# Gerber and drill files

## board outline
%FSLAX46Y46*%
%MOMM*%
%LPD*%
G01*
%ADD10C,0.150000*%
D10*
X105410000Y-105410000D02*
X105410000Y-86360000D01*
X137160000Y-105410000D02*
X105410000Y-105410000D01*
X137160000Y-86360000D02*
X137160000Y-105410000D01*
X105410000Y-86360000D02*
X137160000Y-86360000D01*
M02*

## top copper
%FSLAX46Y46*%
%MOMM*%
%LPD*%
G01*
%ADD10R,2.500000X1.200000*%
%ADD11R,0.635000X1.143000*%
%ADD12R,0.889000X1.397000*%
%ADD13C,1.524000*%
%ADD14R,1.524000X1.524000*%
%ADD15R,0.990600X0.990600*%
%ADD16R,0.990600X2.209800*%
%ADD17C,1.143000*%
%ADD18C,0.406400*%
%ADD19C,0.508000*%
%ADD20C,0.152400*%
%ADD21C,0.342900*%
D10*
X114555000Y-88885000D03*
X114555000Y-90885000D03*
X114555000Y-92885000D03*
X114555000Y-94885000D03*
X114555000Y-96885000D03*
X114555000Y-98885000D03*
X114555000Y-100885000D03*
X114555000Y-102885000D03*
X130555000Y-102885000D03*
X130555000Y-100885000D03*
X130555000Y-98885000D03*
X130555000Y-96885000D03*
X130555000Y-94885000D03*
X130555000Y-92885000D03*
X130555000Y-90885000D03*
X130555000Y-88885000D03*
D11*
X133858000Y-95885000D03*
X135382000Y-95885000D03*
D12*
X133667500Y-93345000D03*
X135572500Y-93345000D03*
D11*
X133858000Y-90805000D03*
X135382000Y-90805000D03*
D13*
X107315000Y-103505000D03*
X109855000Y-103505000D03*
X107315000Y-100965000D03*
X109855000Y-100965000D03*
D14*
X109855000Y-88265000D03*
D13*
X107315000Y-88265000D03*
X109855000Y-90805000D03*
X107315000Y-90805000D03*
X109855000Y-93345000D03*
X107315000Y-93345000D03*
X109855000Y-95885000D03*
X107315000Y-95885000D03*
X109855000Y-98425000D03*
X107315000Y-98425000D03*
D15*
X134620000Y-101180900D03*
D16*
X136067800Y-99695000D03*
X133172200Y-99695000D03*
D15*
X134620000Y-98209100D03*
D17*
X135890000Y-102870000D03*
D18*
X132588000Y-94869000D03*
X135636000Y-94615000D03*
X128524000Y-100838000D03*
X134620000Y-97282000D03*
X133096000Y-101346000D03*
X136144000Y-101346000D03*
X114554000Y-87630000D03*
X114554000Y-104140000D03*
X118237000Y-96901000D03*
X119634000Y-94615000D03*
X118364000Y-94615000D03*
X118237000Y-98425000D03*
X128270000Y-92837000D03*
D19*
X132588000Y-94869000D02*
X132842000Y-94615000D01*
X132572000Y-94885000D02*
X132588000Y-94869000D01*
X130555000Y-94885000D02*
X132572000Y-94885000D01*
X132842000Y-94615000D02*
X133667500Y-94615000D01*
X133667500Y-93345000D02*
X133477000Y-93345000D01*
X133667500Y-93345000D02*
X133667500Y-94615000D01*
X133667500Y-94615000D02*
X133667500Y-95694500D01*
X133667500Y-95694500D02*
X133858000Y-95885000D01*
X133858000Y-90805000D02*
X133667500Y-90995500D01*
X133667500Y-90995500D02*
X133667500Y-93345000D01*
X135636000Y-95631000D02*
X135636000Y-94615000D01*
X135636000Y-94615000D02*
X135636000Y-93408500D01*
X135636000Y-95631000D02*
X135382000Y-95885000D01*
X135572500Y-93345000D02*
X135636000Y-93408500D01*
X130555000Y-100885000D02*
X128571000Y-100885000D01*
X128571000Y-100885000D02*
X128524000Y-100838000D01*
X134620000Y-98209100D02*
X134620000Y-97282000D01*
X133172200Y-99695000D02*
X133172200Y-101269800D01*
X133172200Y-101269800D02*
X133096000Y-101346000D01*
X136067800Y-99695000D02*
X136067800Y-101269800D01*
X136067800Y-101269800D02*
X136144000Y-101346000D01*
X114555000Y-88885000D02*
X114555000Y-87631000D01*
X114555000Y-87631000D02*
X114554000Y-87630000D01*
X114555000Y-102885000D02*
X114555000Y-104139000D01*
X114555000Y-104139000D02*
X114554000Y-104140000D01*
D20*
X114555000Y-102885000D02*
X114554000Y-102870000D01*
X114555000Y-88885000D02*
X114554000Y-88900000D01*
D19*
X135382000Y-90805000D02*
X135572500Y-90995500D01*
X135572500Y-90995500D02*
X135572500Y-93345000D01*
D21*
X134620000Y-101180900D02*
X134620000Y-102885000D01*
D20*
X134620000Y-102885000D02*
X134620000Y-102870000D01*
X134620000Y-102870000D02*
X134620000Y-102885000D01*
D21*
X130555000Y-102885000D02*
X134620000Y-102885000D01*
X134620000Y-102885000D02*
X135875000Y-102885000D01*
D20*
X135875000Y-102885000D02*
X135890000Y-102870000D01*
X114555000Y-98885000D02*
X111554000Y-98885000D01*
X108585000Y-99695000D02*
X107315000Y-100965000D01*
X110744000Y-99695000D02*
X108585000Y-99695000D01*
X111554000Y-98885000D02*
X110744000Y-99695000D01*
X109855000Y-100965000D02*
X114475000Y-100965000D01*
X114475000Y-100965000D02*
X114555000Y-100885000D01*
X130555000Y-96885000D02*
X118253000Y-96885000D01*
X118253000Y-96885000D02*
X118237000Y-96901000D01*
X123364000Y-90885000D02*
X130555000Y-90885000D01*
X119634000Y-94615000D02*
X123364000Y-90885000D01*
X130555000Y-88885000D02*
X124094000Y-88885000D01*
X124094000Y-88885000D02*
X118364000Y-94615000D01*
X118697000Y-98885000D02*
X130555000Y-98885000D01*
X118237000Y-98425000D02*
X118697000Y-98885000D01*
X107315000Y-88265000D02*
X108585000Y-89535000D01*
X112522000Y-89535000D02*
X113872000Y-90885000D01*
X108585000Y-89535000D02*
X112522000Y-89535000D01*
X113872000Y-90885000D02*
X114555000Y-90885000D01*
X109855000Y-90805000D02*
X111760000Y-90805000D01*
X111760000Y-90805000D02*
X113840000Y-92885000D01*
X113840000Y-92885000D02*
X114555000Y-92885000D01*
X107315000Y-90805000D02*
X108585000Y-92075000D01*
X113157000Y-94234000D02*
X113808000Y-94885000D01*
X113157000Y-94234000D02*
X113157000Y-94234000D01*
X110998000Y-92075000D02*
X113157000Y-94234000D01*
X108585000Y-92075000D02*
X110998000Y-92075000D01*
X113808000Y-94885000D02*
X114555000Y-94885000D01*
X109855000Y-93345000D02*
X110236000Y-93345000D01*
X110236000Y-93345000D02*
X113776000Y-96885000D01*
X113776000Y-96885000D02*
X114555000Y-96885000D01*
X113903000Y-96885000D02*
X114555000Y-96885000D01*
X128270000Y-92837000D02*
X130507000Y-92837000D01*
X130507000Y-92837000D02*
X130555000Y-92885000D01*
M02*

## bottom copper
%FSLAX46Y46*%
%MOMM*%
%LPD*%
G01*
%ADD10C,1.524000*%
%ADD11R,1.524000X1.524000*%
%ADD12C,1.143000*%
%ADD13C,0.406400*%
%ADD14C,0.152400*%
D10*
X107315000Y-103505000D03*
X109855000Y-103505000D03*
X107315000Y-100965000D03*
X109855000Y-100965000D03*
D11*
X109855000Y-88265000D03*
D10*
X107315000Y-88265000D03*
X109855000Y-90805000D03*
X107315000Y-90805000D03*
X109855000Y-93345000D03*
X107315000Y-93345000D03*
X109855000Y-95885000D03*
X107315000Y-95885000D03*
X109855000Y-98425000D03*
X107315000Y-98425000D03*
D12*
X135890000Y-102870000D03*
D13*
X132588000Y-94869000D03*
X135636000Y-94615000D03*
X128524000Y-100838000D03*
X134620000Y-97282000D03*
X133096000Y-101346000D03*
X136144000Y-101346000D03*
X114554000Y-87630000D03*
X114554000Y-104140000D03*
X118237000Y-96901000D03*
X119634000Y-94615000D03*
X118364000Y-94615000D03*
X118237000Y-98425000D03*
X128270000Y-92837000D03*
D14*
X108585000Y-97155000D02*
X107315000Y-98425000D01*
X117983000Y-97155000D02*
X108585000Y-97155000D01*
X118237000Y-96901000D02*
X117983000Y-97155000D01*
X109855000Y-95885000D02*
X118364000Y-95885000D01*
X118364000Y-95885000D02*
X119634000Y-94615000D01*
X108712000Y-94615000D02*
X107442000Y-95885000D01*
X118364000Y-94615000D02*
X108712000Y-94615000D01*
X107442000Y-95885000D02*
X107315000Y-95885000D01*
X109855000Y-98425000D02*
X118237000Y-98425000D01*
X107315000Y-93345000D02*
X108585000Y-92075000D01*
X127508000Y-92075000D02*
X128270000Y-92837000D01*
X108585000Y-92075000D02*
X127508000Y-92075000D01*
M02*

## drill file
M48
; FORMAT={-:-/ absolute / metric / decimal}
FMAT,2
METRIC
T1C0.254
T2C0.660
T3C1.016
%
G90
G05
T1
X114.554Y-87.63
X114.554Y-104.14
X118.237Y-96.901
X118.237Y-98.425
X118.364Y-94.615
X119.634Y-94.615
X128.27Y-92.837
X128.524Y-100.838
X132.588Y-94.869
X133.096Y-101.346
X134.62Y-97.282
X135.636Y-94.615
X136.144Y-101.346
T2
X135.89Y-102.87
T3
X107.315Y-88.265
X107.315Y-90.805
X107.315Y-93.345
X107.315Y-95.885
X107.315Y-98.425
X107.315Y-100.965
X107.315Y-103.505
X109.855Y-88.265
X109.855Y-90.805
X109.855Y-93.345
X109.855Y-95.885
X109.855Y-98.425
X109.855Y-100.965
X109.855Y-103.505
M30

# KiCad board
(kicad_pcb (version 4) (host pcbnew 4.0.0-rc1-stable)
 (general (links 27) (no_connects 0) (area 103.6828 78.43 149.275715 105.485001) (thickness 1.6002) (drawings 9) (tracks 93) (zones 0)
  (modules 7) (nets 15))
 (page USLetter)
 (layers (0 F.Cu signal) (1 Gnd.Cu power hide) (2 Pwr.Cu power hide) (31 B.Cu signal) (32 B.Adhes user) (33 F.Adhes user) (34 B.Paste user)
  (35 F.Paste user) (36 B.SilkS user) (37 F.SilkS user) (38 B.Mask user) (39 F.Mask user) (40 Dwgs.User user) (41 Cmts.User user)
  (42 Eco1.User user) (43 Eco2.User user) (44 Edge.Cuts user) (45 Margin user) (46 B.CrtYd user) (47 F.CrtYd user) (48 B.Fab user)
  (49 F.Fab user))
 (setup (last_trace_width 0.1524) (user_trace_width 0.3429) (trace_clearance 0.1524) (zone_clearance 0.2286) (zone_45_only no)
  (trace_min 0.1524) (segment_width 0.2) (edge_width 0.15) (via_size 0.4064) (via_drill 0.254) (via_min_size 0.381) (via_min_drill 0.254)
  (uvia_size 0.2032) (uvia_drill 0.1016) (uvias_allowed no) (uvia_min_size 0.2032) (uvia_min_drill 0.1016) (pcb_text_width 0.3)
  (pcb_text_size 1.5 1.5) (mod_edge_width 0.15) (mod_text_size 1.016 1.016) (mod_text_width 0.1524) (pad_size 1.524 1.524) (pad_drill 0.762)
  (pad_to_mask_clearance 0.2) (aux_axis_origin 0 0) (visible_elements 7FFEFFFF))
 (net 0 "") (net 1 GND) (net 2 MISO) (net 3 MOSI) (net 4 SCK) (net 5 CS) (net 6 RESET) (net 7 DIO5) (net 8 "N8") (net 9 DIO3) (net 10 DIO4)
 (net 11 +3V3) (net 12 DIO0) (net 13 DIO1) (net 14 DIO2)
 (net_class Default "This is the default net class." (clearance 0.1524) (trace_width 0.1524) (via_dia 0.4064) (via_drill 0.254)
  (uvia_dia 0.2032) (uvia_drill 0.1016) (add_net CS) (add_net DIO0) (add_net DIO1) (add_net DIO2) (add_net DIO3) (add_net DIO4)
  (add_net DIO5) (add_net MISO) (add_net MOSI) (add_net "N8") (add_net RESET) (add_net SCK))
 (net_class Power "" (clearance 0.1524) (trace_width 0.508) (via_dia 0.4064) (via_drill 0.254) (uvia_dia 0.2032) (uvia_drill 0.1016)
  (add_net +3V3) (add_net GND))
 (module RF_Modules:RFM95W (layer F.Cu) (at 122.555 95.885)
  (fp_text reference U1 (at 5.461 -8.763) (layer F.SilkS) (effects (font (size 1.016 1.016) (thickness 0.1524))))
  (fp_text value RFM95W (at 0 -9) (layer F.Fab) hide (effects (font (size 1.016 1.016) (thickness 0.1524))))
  (pad 1 smd rect (at -8 -7) (size 2.5 1.2) (layers F.Cu F.Paste F.Mask) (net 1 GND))
  (pad 2 smd rect (at -8 -5) (size 2.5 1.2) (layers F.Cu F.Paste F.Mask) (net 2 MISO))
  (pad 3 smd rect (at -8 -3) (size 2.5 1.2) (layers F.Cu F.Paste F.Mask) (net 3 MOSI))
  (pad 4 smd rect (at -8 -1) (size 2.5 1.2) (layers F.Cu F.Paste F.Mask) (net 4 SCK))
  (pad 5 smd rect (at -8 1) (size 2.5 1.2) (layers F.Cu F.Paste F.Mask) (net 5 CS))
  (pad 6 smd rect (at -8 3) (size 2.5 1.2) (layers F.Cu F.Paste F.Mask) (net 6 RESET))
  (pad 7 smd rect (at -8 5) (size 2.5 1.2) (layers F.Cu F.Paste F.Mask) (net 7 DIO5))
  (pad 8 smd rect (at -8 7) (size 2.5 1.2) (layers F.Cu F.Paste F.Mask) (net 1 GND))
  (pad 9 smd rect (at 8 7) (size 2.5 1.2) (layers F.Cu F.Paste F.Mask) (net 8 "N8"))
  (pad 10 smd rect (at 8 5) (size 2.5 1.2) (layers F.Cu F.Paste F.Mask) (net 1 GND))
  (pad 11 smd rect (at 8 3) (size 2.5 1.2) (layers F.Cu F.Paste F.Mask) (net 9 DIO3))
  (pad 12 smd rect (at 8 1) (size 2.5 1.2) (layers F.Cu F.Paste F.Mask) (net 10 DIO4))
  (pad 13 smd rect (at 8 -1) (size 2.5 1.2) (layers F.Cu F.Paste F.Mask) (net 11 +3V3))
  (pad 14 smd rect (at 8 -3) (size 2.5 1.2) (layers F.Cu F.Paste F.Mask) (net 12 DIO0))
  (pad 15 smd rect (at 8 -5) (size 2.5 1.2) (layers F.Cu F.Paste F.Mask) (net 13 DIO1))
  (pad 16 smd rect (at 8 -7) (size 2.5 1.2) (layers F.Cu F.Paste F.Mask) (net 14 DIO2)))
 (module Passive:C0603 (layer F.Cu) (at 134.62 95.885)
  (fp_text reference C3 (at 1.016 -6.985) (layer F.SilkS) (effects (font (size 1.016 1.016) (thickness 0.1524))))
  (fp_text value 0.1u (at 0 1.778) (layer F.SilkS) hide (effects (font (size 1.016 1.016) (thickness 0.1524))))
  (pad 1 smd rect (at -0.762 0) (size 0.635 1.143) (layers F.Cu F.Paste F.Mask) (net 11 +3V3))
  (pad 2 smd rect (at 0.762 0) (size 0.635 1.143) (layers F.Cu F.Paste F.Mask) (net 1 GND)))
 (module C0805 (layer F.Cu) (at 134.62 93.345)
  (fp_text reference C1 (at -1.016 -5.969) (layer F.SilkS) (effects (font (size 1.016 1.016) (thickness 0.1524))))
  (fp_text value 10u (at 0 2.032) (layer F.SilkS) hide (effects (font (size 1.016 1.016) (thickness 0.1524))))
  (pad 1 smd rect (at -0.9525 0) (size 0.889 1.397) (layers F.Cu F.Paste F.Mask) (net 11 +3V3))
  (pad 2 smd rect (at 0.9525 0) (size 0.889 1.397) (layers F.Cu F.Paste F.Mask) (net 1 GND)))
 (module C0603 (layer F.Cu) (at 134.62 90.805)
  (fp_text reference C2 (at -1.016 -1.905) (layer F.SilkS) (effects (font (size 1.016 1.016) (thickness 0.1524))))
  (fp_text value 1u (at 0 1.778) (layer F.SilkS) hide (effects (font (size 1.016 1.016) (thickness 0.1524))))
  (pad 1 smd rect (at -0.762 0) (size 0.635 1.143) (layers F.Cu F.Paste F.Mask) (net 11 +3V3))
  (pad 2 smd rect (at 0.762 0) (size 0.635 1.143) (layers F.Cu F.Paste F.Mask) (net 1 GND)))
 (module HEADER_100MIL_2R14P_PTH (layer B.Cu) (at 108.585 95.885 270)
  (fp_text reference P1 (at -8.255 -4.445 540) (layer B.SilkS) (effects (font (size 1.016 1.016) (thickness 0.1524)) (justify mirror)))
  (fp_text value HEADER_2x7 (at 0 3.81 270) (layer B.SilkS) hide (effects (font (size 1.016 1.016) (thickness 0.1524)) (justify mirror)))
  (pad 14 thru_hole circle (at 7.62 1.27 270) (size 1.524 1.524) (drill 1.016) (layers *.Cu *.Mask B.SilkS) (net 1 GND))
  (pad 13 thru_hole circle (at 7.62 -1.27 270) (size 1.524 1.524) (drill 1.016) (layers *.Cu *.Mask B.SilkS) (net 11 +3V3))
  (pad 12 thru_hole circle (at 5.08 1.27 270) (size 1.524 1.524) (drill 1.016) (layers *.Cu *.Mask B.SilkS) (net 6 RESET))
  (pad 11 thru_hole circle (at 5.08 -1.27 270) (size 1.524 1.524) (drill 1.016) (layers *.Cu *.Mask B.SilkS) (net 7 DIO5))
  (pad 1 thru_hole rect (at -7.62 -1.27 270) (size 1.524 1.524) (drill 1.016) (layers *.Cu *.Mask B.SilkS) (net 1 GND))
  (pad 2 thru_hole circle (at -7.62 1.27 270) (size 1.524 1.524) (drill 1.016) (layers *.Cu *.Mask B.SilkS) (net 2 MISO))
  (pad 3 thru_hole circle (at -5.08 -1.27 270) (size 1.524 1.524) (drill 1.016) (layers *.Cu *.Mask B.SilkS) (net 3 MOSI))
  (pad 4 thru_hole circle (at -5.08 1.27 270) (size 1.524 1.524) (drill 1.016) (layers *.Cu *.Mask B.SilkS) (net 4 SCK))
  (pad 5 thru_hole circle (at -2.54 -1.27 270) (size 1.524 1.524) (drill 1.016) (layers *.Cu *.Mask B.SilkS) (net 5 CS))
  (pad 6 thru_hole circle (at -2.54 1.27 270) (size 1.524 1.524) (drill 1.016) (layers *.Cu *.Mask B.SilkS) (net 12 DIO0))
  (pad 7 thru_hole circle (at 0 -1.27 270) (size 1.524 1.524) (drill 1.016) (layers *.Cu *.Mask B.SilkS) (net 13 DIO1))
  (pad 8 thru_hole circle (at 0 1.27 270) (size 1.524 1.524) (drill 1.016) (layers *.Cu *.Mask B.SilkS) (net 14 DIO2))
  (pad 9 thru_hole circle (at 2.54 -1.27 270) (size 1.524 1.524) (drill 1.016) (layers *.Cu *.Mask B.SilkS) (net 9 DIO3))
  (pad 10 thru_hole circle (at 2.54 1.27 270) (size 1.524 1.524) (drill 1.016) (layers *.Cu *.Mask B.SilkS) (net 10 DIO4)))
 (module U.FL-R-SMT (layer F.Cu) (at 134.62 99.695)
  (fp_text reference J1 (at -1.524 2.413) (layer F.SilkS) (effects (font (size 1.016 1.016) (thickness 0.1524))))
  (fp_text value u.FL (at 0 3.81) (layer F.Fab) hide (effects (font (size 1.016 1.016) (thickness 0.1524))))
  (pad 1 smd rect (at 0 1.4859) (size 0.9906 0.9906) (layers F.Cu F.Paste F.Mask) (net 8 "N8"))
  (pad 4 smd rect (at 1.4478 0) (size 0.9906 2.2098) (layers F.Cu F.Paste F.Mask) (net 1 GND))
  (pad 2 smd rect (at -1.4478 0) (size 0.9906 2.2098) (layers F.Cu F.Paste F.Mask) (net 1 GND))
  (pad 3 smd rect (at 0 -1.4859) (size 0.9906 0.9906) (layers F.Cu F.Paste F.Mask) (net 1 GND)))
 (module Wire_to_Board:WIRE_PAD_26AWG (layer F.Cu) (at 135.89 102.87)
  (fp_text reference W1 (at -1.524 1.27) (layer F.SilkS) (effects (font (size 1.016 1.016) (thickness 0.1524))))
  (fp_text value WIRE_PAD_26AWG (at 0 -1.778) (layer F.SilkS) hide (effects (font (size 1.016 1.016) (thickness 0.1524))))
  (pad 1 thru_hole circle (at 0 0) (size 1.143 1.143) (drill 0.6604) (layers *.Cu *.Mask F.SilkS) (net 8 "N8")))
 (gr_line (start 105.41 105.41) (end 105.41 86.36) (angle 90) (layer Edge.Cuts) (width 0.15))
 (gr_line (start 137.16 105.41) (end 105.41 105.41) (angle 90) (layer Edge.Cuts) (width 0.15))
 (gr_line (start 137.16 86.36) (end 137.16 105.41) (angle 90) (layer Edge.Cuts) (width 0.15))
 (gr_line (start 105.41 86.36) (end 137.16 86.36) (angle 90) (layer Edge.Cuts) (width 0.15))
 (segment (start 132.588 94.869) (end 132.842 94.615) (width 0.508) (layer F.Cu) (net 11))
 (segment (start 132.572 94.885) (end 132.588 94.869) (width 0.508) (layer F.Cu) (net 11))
 (via (at 132.588 94.869) (size 0.4064) (drill 0.254) (layers F.Cu B.Cu) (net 11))
 (segment (start 130.555 94.885) (end 132.572 94.885) (width 0.508) (layer F.Cu) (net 11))
 (segment (start 132.842 94.615) (end 133.6675 94.615) (width 0.508) (layer F.Cu) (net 11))
 (segment (start 133.6675 93.345) (end 133.477 93.345) (width 0.508) (layer F.Cu) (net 11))
 (segment (start 133.6675 93.345) (end 133.6675 94.615) (width 0.508) (layer F.Cu) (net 11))
 (segment (start 133.6675 94.615) (end 133.6675 95.6945) (width 0.508) (layer F.Cu) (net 11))
 (segment (start 133.6675 95.6945) (end 133.858 95.885) (width 0.508) (layer F.Cu) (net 11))
 (segment (start 133.858 90.805) (end 133.6675 90.9955) (width 0.508) (layer F.Cu) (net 11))
 (segment (start 133.6675 90.9955) (end 133.6675 93.345) (width 0.508) (layer F.Cu) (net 11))
 (segment (start 135.636 95.631) (end 135.636 94.615) (width 0.508) (layer F.Cu) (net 1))
 (via (at 135.636 94.615) (size 0.4064) (drill 0.254) (layers F.Cu B.Cu) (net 1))
 (segment (start 135.636 94.615) (end 135.636 93.4085) (width 0.508) (layer F.Cu) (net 1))
 (segment (start 135.636 95.631) (end 135.382 95.885) (width 0.508) (layer F.Cu) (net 1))
 (segment (start 135.5725 93.345) (end 135.636 93.4085) (width 0.508) (layer F.Cu) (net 1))
 (segment (start 130.555 100.885) (end 128.571 100.885) (width 0.508) (layer F.Cu) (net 1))
 (via (at 128.524 100.838) (size 0.4064) (drill 0.254) (layers F.Cu B.Cu) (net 1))
 (segment (start 128.571 100.885) (end 128.524 100.838) (width 0.508) (layer F.Cu) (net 1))
 (segment (start 134.62 98.2091) (end 134.62 97.282) (width 0.508) (layer F.Cu) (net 1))
 (via (at 134.62 97.282) (size 0.4064) (drill 0.254) (layers F.Cu B.Cu) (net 1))
 (segment (start 133.1722 99.695) (end 133.1722 101.2698) (width 0.508) (layer F.Cu) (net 1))
 (via (at 133.096 101.346) (size 0.4064) (drill 0.254) (layers F.Cu B.Cu) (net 1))
 (segment (start 133.1722 101.2698) (end 133.096 101.346) (width 0.508) (layer F.Cu) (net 1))
 (segment (start 136.0678 99.695) (end 136.0678 101.2698) (width 0.508) (layer F.Cu) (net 1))
 (via (at 136.144 101.346) (size 0.4064) (drill 0.254) (layers F.Cu B.Cu) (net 1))
 (segment (start 136.0678 101.2698) (end 136.144 101.346) (width 0.508) (layer F.Cu) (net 1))
 (segment (start 114.555 88.885) (end 114.555 87.631) (width 0.508) (layer F.Cu) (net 1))
 (via (at 114.554 87.63) (size 0.4064) (drill 0.254) (layers F.Cu B.Cu) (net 1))
 (segment (start 114.555 87.631) (end 114.554 87.63) (width 0.508) (layer F.Cu) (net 1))
 (segment (start 114.555 102.885) (end 114.555 104.139) (width 0.508) (layer F.Cu) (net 1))
 (via (at 114.554 104.14) (size 0.4064) (drill 0.254) (layers F.Cu B.Cu) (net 1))
 (segment (start 114.555 104.139) (end 114.554 104.14) (width 0.508) (layer F.Cu) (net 1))
 (segment (start 114.555 102.885) (end 114.554 102.87) (width 0.1524) (layer F.Cu) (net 1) (status 80000))
 (segment (start 114.555 88.885) (end 114.554 88.9) (width 0.1524) (layer F.Cu) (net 1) (status 80000))
 (segment (start 135.382 90.805) (end 135.5725 90.9955) (width 0.508) (layer F.Cu) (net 1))
 (segment (start 135.5725 90.9955) (end 135.5725 93.345) (width 0.508) (layer F.Cu) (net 1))
 (segment (start 134.62 101.1809) (end 134.62 102.885) (width 0.3429) (layer F.Cu) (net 8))
 (segment (start 134.62 102.885) (end 134.62 102.87) (width 0.1524) (layer F.Cu) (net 8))
 (segment (start 134.62 102.87) (end 134.62 102.885) (width 0.1524) (layer F.Cu) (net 8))
 (segment (start 130.555 102.885) (end 134.62 102.885) (width 0.3429) (layer F.Cu) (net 8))
 (segment (start 134.62 102.885) (end 135.875 102.885) (width 0.3429) (layer F.Cu) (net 8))
 (segment (start 135.875 102.885) (end 135.89 102.87) (width 0.1524) (layer F.Cu) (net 8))
 (segment (start 114.555 98.885) (end 111.554 98.885) (width 0.1524) (layer F.Cu) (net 6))
 (segment (start 108.585 99.695) (end 107.315 100.965) (width 0.1524) (layer F.Cu) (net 6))
 (segment (start 110.744 99.695) (end 108.585 99.695) (width 0.1524) (layer F.Cu) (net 6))
 (segment (start 111.554 98.885) (end 110.744 99.695) (width 0.1524) (layer F.Cu) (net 6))
 (segment (start 109.855 100.965) (end 114.475 100.965) (width 0.1524) (layer F.Cu) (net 7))
 (segment (start 114.475 100.965) (end 114.555 100.885) (width 0.1524) (layer F.Cu) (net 7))
 (segment (start 130.555 96.885) (end 118.253 96.885) (width 0.1524) (layer F.Cu) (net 10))
 (segment (start 108.585 97.155) (end 107.315 98.425) (width 0.1524) (layer B.Cu) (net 10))
 (segment (start 117.983 97.155) (end 108.585 97.155) (width 0.1524) (layer B.Cu) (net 10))
 (segment (start 118.237 96.901) (end 117.983 97.155) (width 0.1524) (layer B.Cu) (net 10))
 (via (at 118.237 96.901) (size 0.4064) (drill 0.254) (layers F.Cu B.Cu) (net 10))
 (segment (start 118.253 96.885) (end 118.237 96.901) (width 0.1524) (layer F.Cu) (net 10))
 (segment (start 109.855 95.885) (end 118.364 95.885) (width 0.1524) (layer B.Cu) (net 13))
 (segment (start 123.364 90.885) (end 130.555 90.885) (width 0.1524) (layer F.Cu) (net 13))
 (segment (start 119.634 94.615) (end 123.364 90.885) (width 0.1524) (layer F.Cu) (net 13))
 (via (at 119.634 94.615) (size 0.4064) (drill 0.254) (layers F.Cu B.Cu) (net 13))
 (segment (start 118.364 95.885) (end 119.634 94.615) (width 0.1524) (layer B.Cu) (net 13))
 (segment (start 130.555 88.885) (end 124.094 88.885) (width 0.1524) (layer F.Cu) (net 14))
 (segment (start 108.712 94.615) (end 107.442 95.885) (width 0.1524) (layer B.Cu) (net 14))
 (segment (start 118.364 94.615) (end 108.712 94.615) (width 0.1524) (layer B.Cu) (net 14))
 (via (at 118.364 94.615) (size 0.4064) (drill 0.254) (layers F.Cu B.Cu) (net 14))
 (segment (start 124.094 88.885) (end 118.364 94.615) (width 0.1524) (layer F.Cu) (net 14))
 (segment (start 107.442 95.885) (end 107.315 95.885) (width 0.1524) (layer B.Cu) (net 14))
 (segment (start 109.855 98.425) (end 118.237 98.425) (width 0.1524) (layer B.Cu) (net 9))
 (segment (start 118.697 98.885) (end 130.555 98.885) (width 0.1524) (layer F.Cu) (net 9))
 (segment (start 118.237 98.425) (end 118.697 98.885) (width 0.1524) (layer F.Cu) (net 9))
 (via (at 118.237 98.425) (size 0.4064) (drill 0.254) (layers F.Cu B.Cu) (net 9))
 (segment (start 107.315 88.265) (end 108.585 89.535) (width 0.1524) (layer F.Cu) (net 2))
 (segment (start 112.522 89.535) (end 113.872 90.885) (width 0.1524) (layer F.Cu) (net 2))
 (segment (start 108.585 89.535) (end 112.522 89.535) (width 0.1524) (layer F.Cu) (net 2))
 (segment (start 113.872 90.885) (end 114.555 90.885) (width 0.1524) (layer F.Cu) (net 2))
 (segment (start 109.855 90.805) (end 111.76 90.805) (width 0.1524) (layer F.Cu) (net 3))
 (segment (start 111.76 90.805) (end 113.84 92.885) (width 0.1524) (layer F.Cu) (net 3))
 (segment (start 113.84 92.885) (end 114.555 92.885) (width 0.1524) (layer F.Cu) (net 3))
 (segment (start 107.315 90.805) (end 108.585 92.075) (width 0.1524) (layer F.Cu) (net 4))
 (segment (start 113.157 94.234) (end 113.808 94.885) (width 0.1524) (layer F.Cu) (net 4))
 (segment (start 113.157 94.234) (end 113.157 94.234) (width 0.1524) (layer F.Cu) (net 4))
 (segment (start 110.998 92.075) (end 113.157 94.234) (width 0.1524) (layer F.Cu) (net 4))
 (segment (start 108.585 92.075) (end 110.998 92.075) (width 0.1524) (layer F.Cu) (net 4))
 (segment (start 113.808 94.885) (end 114.555 94.885) (width 0.1524) (layer F.Cu) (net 4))
 (segment (start 109.855 93.345) (end 110.236 93.345) (width 0.1524) (layer F.Cu) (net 5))
 (segment (start 110.236 93.345) (end 113.776 96.885) (width 0.1524) (layer F.Cu) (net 5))
 (segment (start 113.776 96.885) (end 114.555 96.885) (width 0.1524) (layer F.Cu) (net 5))
 (segment (start 113.903 96.885) (end 114.555 96.885) (width 0.1524) (layer F.Cu) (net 5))
 (segment (start 107.315 93.345) (end 108.585 92.075) (width 0.1524) (layer B.Cu) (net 12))
 (segment (start 128.27 92.837) (end 130.507 92.837) (width 0.1524) (layer F.Cu) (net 12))
 (via (at 128.27 92.837) (size 0.4064) (drill 0.254) (layers F.Cu B.Cu) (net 12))
 (segment (start 127.508 92.075) (end 128.27 92.837) (width 0.1524) (layer B.Cu) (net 12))
 (segment (start 108.585 92.075) (end 127.508 92.075) (width 0.1524) (layer B.Cu) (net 12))
 (segment (start 130.507 92.837) (end 130.555 92.885) (width 0.1524) (layer F.Cu) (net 12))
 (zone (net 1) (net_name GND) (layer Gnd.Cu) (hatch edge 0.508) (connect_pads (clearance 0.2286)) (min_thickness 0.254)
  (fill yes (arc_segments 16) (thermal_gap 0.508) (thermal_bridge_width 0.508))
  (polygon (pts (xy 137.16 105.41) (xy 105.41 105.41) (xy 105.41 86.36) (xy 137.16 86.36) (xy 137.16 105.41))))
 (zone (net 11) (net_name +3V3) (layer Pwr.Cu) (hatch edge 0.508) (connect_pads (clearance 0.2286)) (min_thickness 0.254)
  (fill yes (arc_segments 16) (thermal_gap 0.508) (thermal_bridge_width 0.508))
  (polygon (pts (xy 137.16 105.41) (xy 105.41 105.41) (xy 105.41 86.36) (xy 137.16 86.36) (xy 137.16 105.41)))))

